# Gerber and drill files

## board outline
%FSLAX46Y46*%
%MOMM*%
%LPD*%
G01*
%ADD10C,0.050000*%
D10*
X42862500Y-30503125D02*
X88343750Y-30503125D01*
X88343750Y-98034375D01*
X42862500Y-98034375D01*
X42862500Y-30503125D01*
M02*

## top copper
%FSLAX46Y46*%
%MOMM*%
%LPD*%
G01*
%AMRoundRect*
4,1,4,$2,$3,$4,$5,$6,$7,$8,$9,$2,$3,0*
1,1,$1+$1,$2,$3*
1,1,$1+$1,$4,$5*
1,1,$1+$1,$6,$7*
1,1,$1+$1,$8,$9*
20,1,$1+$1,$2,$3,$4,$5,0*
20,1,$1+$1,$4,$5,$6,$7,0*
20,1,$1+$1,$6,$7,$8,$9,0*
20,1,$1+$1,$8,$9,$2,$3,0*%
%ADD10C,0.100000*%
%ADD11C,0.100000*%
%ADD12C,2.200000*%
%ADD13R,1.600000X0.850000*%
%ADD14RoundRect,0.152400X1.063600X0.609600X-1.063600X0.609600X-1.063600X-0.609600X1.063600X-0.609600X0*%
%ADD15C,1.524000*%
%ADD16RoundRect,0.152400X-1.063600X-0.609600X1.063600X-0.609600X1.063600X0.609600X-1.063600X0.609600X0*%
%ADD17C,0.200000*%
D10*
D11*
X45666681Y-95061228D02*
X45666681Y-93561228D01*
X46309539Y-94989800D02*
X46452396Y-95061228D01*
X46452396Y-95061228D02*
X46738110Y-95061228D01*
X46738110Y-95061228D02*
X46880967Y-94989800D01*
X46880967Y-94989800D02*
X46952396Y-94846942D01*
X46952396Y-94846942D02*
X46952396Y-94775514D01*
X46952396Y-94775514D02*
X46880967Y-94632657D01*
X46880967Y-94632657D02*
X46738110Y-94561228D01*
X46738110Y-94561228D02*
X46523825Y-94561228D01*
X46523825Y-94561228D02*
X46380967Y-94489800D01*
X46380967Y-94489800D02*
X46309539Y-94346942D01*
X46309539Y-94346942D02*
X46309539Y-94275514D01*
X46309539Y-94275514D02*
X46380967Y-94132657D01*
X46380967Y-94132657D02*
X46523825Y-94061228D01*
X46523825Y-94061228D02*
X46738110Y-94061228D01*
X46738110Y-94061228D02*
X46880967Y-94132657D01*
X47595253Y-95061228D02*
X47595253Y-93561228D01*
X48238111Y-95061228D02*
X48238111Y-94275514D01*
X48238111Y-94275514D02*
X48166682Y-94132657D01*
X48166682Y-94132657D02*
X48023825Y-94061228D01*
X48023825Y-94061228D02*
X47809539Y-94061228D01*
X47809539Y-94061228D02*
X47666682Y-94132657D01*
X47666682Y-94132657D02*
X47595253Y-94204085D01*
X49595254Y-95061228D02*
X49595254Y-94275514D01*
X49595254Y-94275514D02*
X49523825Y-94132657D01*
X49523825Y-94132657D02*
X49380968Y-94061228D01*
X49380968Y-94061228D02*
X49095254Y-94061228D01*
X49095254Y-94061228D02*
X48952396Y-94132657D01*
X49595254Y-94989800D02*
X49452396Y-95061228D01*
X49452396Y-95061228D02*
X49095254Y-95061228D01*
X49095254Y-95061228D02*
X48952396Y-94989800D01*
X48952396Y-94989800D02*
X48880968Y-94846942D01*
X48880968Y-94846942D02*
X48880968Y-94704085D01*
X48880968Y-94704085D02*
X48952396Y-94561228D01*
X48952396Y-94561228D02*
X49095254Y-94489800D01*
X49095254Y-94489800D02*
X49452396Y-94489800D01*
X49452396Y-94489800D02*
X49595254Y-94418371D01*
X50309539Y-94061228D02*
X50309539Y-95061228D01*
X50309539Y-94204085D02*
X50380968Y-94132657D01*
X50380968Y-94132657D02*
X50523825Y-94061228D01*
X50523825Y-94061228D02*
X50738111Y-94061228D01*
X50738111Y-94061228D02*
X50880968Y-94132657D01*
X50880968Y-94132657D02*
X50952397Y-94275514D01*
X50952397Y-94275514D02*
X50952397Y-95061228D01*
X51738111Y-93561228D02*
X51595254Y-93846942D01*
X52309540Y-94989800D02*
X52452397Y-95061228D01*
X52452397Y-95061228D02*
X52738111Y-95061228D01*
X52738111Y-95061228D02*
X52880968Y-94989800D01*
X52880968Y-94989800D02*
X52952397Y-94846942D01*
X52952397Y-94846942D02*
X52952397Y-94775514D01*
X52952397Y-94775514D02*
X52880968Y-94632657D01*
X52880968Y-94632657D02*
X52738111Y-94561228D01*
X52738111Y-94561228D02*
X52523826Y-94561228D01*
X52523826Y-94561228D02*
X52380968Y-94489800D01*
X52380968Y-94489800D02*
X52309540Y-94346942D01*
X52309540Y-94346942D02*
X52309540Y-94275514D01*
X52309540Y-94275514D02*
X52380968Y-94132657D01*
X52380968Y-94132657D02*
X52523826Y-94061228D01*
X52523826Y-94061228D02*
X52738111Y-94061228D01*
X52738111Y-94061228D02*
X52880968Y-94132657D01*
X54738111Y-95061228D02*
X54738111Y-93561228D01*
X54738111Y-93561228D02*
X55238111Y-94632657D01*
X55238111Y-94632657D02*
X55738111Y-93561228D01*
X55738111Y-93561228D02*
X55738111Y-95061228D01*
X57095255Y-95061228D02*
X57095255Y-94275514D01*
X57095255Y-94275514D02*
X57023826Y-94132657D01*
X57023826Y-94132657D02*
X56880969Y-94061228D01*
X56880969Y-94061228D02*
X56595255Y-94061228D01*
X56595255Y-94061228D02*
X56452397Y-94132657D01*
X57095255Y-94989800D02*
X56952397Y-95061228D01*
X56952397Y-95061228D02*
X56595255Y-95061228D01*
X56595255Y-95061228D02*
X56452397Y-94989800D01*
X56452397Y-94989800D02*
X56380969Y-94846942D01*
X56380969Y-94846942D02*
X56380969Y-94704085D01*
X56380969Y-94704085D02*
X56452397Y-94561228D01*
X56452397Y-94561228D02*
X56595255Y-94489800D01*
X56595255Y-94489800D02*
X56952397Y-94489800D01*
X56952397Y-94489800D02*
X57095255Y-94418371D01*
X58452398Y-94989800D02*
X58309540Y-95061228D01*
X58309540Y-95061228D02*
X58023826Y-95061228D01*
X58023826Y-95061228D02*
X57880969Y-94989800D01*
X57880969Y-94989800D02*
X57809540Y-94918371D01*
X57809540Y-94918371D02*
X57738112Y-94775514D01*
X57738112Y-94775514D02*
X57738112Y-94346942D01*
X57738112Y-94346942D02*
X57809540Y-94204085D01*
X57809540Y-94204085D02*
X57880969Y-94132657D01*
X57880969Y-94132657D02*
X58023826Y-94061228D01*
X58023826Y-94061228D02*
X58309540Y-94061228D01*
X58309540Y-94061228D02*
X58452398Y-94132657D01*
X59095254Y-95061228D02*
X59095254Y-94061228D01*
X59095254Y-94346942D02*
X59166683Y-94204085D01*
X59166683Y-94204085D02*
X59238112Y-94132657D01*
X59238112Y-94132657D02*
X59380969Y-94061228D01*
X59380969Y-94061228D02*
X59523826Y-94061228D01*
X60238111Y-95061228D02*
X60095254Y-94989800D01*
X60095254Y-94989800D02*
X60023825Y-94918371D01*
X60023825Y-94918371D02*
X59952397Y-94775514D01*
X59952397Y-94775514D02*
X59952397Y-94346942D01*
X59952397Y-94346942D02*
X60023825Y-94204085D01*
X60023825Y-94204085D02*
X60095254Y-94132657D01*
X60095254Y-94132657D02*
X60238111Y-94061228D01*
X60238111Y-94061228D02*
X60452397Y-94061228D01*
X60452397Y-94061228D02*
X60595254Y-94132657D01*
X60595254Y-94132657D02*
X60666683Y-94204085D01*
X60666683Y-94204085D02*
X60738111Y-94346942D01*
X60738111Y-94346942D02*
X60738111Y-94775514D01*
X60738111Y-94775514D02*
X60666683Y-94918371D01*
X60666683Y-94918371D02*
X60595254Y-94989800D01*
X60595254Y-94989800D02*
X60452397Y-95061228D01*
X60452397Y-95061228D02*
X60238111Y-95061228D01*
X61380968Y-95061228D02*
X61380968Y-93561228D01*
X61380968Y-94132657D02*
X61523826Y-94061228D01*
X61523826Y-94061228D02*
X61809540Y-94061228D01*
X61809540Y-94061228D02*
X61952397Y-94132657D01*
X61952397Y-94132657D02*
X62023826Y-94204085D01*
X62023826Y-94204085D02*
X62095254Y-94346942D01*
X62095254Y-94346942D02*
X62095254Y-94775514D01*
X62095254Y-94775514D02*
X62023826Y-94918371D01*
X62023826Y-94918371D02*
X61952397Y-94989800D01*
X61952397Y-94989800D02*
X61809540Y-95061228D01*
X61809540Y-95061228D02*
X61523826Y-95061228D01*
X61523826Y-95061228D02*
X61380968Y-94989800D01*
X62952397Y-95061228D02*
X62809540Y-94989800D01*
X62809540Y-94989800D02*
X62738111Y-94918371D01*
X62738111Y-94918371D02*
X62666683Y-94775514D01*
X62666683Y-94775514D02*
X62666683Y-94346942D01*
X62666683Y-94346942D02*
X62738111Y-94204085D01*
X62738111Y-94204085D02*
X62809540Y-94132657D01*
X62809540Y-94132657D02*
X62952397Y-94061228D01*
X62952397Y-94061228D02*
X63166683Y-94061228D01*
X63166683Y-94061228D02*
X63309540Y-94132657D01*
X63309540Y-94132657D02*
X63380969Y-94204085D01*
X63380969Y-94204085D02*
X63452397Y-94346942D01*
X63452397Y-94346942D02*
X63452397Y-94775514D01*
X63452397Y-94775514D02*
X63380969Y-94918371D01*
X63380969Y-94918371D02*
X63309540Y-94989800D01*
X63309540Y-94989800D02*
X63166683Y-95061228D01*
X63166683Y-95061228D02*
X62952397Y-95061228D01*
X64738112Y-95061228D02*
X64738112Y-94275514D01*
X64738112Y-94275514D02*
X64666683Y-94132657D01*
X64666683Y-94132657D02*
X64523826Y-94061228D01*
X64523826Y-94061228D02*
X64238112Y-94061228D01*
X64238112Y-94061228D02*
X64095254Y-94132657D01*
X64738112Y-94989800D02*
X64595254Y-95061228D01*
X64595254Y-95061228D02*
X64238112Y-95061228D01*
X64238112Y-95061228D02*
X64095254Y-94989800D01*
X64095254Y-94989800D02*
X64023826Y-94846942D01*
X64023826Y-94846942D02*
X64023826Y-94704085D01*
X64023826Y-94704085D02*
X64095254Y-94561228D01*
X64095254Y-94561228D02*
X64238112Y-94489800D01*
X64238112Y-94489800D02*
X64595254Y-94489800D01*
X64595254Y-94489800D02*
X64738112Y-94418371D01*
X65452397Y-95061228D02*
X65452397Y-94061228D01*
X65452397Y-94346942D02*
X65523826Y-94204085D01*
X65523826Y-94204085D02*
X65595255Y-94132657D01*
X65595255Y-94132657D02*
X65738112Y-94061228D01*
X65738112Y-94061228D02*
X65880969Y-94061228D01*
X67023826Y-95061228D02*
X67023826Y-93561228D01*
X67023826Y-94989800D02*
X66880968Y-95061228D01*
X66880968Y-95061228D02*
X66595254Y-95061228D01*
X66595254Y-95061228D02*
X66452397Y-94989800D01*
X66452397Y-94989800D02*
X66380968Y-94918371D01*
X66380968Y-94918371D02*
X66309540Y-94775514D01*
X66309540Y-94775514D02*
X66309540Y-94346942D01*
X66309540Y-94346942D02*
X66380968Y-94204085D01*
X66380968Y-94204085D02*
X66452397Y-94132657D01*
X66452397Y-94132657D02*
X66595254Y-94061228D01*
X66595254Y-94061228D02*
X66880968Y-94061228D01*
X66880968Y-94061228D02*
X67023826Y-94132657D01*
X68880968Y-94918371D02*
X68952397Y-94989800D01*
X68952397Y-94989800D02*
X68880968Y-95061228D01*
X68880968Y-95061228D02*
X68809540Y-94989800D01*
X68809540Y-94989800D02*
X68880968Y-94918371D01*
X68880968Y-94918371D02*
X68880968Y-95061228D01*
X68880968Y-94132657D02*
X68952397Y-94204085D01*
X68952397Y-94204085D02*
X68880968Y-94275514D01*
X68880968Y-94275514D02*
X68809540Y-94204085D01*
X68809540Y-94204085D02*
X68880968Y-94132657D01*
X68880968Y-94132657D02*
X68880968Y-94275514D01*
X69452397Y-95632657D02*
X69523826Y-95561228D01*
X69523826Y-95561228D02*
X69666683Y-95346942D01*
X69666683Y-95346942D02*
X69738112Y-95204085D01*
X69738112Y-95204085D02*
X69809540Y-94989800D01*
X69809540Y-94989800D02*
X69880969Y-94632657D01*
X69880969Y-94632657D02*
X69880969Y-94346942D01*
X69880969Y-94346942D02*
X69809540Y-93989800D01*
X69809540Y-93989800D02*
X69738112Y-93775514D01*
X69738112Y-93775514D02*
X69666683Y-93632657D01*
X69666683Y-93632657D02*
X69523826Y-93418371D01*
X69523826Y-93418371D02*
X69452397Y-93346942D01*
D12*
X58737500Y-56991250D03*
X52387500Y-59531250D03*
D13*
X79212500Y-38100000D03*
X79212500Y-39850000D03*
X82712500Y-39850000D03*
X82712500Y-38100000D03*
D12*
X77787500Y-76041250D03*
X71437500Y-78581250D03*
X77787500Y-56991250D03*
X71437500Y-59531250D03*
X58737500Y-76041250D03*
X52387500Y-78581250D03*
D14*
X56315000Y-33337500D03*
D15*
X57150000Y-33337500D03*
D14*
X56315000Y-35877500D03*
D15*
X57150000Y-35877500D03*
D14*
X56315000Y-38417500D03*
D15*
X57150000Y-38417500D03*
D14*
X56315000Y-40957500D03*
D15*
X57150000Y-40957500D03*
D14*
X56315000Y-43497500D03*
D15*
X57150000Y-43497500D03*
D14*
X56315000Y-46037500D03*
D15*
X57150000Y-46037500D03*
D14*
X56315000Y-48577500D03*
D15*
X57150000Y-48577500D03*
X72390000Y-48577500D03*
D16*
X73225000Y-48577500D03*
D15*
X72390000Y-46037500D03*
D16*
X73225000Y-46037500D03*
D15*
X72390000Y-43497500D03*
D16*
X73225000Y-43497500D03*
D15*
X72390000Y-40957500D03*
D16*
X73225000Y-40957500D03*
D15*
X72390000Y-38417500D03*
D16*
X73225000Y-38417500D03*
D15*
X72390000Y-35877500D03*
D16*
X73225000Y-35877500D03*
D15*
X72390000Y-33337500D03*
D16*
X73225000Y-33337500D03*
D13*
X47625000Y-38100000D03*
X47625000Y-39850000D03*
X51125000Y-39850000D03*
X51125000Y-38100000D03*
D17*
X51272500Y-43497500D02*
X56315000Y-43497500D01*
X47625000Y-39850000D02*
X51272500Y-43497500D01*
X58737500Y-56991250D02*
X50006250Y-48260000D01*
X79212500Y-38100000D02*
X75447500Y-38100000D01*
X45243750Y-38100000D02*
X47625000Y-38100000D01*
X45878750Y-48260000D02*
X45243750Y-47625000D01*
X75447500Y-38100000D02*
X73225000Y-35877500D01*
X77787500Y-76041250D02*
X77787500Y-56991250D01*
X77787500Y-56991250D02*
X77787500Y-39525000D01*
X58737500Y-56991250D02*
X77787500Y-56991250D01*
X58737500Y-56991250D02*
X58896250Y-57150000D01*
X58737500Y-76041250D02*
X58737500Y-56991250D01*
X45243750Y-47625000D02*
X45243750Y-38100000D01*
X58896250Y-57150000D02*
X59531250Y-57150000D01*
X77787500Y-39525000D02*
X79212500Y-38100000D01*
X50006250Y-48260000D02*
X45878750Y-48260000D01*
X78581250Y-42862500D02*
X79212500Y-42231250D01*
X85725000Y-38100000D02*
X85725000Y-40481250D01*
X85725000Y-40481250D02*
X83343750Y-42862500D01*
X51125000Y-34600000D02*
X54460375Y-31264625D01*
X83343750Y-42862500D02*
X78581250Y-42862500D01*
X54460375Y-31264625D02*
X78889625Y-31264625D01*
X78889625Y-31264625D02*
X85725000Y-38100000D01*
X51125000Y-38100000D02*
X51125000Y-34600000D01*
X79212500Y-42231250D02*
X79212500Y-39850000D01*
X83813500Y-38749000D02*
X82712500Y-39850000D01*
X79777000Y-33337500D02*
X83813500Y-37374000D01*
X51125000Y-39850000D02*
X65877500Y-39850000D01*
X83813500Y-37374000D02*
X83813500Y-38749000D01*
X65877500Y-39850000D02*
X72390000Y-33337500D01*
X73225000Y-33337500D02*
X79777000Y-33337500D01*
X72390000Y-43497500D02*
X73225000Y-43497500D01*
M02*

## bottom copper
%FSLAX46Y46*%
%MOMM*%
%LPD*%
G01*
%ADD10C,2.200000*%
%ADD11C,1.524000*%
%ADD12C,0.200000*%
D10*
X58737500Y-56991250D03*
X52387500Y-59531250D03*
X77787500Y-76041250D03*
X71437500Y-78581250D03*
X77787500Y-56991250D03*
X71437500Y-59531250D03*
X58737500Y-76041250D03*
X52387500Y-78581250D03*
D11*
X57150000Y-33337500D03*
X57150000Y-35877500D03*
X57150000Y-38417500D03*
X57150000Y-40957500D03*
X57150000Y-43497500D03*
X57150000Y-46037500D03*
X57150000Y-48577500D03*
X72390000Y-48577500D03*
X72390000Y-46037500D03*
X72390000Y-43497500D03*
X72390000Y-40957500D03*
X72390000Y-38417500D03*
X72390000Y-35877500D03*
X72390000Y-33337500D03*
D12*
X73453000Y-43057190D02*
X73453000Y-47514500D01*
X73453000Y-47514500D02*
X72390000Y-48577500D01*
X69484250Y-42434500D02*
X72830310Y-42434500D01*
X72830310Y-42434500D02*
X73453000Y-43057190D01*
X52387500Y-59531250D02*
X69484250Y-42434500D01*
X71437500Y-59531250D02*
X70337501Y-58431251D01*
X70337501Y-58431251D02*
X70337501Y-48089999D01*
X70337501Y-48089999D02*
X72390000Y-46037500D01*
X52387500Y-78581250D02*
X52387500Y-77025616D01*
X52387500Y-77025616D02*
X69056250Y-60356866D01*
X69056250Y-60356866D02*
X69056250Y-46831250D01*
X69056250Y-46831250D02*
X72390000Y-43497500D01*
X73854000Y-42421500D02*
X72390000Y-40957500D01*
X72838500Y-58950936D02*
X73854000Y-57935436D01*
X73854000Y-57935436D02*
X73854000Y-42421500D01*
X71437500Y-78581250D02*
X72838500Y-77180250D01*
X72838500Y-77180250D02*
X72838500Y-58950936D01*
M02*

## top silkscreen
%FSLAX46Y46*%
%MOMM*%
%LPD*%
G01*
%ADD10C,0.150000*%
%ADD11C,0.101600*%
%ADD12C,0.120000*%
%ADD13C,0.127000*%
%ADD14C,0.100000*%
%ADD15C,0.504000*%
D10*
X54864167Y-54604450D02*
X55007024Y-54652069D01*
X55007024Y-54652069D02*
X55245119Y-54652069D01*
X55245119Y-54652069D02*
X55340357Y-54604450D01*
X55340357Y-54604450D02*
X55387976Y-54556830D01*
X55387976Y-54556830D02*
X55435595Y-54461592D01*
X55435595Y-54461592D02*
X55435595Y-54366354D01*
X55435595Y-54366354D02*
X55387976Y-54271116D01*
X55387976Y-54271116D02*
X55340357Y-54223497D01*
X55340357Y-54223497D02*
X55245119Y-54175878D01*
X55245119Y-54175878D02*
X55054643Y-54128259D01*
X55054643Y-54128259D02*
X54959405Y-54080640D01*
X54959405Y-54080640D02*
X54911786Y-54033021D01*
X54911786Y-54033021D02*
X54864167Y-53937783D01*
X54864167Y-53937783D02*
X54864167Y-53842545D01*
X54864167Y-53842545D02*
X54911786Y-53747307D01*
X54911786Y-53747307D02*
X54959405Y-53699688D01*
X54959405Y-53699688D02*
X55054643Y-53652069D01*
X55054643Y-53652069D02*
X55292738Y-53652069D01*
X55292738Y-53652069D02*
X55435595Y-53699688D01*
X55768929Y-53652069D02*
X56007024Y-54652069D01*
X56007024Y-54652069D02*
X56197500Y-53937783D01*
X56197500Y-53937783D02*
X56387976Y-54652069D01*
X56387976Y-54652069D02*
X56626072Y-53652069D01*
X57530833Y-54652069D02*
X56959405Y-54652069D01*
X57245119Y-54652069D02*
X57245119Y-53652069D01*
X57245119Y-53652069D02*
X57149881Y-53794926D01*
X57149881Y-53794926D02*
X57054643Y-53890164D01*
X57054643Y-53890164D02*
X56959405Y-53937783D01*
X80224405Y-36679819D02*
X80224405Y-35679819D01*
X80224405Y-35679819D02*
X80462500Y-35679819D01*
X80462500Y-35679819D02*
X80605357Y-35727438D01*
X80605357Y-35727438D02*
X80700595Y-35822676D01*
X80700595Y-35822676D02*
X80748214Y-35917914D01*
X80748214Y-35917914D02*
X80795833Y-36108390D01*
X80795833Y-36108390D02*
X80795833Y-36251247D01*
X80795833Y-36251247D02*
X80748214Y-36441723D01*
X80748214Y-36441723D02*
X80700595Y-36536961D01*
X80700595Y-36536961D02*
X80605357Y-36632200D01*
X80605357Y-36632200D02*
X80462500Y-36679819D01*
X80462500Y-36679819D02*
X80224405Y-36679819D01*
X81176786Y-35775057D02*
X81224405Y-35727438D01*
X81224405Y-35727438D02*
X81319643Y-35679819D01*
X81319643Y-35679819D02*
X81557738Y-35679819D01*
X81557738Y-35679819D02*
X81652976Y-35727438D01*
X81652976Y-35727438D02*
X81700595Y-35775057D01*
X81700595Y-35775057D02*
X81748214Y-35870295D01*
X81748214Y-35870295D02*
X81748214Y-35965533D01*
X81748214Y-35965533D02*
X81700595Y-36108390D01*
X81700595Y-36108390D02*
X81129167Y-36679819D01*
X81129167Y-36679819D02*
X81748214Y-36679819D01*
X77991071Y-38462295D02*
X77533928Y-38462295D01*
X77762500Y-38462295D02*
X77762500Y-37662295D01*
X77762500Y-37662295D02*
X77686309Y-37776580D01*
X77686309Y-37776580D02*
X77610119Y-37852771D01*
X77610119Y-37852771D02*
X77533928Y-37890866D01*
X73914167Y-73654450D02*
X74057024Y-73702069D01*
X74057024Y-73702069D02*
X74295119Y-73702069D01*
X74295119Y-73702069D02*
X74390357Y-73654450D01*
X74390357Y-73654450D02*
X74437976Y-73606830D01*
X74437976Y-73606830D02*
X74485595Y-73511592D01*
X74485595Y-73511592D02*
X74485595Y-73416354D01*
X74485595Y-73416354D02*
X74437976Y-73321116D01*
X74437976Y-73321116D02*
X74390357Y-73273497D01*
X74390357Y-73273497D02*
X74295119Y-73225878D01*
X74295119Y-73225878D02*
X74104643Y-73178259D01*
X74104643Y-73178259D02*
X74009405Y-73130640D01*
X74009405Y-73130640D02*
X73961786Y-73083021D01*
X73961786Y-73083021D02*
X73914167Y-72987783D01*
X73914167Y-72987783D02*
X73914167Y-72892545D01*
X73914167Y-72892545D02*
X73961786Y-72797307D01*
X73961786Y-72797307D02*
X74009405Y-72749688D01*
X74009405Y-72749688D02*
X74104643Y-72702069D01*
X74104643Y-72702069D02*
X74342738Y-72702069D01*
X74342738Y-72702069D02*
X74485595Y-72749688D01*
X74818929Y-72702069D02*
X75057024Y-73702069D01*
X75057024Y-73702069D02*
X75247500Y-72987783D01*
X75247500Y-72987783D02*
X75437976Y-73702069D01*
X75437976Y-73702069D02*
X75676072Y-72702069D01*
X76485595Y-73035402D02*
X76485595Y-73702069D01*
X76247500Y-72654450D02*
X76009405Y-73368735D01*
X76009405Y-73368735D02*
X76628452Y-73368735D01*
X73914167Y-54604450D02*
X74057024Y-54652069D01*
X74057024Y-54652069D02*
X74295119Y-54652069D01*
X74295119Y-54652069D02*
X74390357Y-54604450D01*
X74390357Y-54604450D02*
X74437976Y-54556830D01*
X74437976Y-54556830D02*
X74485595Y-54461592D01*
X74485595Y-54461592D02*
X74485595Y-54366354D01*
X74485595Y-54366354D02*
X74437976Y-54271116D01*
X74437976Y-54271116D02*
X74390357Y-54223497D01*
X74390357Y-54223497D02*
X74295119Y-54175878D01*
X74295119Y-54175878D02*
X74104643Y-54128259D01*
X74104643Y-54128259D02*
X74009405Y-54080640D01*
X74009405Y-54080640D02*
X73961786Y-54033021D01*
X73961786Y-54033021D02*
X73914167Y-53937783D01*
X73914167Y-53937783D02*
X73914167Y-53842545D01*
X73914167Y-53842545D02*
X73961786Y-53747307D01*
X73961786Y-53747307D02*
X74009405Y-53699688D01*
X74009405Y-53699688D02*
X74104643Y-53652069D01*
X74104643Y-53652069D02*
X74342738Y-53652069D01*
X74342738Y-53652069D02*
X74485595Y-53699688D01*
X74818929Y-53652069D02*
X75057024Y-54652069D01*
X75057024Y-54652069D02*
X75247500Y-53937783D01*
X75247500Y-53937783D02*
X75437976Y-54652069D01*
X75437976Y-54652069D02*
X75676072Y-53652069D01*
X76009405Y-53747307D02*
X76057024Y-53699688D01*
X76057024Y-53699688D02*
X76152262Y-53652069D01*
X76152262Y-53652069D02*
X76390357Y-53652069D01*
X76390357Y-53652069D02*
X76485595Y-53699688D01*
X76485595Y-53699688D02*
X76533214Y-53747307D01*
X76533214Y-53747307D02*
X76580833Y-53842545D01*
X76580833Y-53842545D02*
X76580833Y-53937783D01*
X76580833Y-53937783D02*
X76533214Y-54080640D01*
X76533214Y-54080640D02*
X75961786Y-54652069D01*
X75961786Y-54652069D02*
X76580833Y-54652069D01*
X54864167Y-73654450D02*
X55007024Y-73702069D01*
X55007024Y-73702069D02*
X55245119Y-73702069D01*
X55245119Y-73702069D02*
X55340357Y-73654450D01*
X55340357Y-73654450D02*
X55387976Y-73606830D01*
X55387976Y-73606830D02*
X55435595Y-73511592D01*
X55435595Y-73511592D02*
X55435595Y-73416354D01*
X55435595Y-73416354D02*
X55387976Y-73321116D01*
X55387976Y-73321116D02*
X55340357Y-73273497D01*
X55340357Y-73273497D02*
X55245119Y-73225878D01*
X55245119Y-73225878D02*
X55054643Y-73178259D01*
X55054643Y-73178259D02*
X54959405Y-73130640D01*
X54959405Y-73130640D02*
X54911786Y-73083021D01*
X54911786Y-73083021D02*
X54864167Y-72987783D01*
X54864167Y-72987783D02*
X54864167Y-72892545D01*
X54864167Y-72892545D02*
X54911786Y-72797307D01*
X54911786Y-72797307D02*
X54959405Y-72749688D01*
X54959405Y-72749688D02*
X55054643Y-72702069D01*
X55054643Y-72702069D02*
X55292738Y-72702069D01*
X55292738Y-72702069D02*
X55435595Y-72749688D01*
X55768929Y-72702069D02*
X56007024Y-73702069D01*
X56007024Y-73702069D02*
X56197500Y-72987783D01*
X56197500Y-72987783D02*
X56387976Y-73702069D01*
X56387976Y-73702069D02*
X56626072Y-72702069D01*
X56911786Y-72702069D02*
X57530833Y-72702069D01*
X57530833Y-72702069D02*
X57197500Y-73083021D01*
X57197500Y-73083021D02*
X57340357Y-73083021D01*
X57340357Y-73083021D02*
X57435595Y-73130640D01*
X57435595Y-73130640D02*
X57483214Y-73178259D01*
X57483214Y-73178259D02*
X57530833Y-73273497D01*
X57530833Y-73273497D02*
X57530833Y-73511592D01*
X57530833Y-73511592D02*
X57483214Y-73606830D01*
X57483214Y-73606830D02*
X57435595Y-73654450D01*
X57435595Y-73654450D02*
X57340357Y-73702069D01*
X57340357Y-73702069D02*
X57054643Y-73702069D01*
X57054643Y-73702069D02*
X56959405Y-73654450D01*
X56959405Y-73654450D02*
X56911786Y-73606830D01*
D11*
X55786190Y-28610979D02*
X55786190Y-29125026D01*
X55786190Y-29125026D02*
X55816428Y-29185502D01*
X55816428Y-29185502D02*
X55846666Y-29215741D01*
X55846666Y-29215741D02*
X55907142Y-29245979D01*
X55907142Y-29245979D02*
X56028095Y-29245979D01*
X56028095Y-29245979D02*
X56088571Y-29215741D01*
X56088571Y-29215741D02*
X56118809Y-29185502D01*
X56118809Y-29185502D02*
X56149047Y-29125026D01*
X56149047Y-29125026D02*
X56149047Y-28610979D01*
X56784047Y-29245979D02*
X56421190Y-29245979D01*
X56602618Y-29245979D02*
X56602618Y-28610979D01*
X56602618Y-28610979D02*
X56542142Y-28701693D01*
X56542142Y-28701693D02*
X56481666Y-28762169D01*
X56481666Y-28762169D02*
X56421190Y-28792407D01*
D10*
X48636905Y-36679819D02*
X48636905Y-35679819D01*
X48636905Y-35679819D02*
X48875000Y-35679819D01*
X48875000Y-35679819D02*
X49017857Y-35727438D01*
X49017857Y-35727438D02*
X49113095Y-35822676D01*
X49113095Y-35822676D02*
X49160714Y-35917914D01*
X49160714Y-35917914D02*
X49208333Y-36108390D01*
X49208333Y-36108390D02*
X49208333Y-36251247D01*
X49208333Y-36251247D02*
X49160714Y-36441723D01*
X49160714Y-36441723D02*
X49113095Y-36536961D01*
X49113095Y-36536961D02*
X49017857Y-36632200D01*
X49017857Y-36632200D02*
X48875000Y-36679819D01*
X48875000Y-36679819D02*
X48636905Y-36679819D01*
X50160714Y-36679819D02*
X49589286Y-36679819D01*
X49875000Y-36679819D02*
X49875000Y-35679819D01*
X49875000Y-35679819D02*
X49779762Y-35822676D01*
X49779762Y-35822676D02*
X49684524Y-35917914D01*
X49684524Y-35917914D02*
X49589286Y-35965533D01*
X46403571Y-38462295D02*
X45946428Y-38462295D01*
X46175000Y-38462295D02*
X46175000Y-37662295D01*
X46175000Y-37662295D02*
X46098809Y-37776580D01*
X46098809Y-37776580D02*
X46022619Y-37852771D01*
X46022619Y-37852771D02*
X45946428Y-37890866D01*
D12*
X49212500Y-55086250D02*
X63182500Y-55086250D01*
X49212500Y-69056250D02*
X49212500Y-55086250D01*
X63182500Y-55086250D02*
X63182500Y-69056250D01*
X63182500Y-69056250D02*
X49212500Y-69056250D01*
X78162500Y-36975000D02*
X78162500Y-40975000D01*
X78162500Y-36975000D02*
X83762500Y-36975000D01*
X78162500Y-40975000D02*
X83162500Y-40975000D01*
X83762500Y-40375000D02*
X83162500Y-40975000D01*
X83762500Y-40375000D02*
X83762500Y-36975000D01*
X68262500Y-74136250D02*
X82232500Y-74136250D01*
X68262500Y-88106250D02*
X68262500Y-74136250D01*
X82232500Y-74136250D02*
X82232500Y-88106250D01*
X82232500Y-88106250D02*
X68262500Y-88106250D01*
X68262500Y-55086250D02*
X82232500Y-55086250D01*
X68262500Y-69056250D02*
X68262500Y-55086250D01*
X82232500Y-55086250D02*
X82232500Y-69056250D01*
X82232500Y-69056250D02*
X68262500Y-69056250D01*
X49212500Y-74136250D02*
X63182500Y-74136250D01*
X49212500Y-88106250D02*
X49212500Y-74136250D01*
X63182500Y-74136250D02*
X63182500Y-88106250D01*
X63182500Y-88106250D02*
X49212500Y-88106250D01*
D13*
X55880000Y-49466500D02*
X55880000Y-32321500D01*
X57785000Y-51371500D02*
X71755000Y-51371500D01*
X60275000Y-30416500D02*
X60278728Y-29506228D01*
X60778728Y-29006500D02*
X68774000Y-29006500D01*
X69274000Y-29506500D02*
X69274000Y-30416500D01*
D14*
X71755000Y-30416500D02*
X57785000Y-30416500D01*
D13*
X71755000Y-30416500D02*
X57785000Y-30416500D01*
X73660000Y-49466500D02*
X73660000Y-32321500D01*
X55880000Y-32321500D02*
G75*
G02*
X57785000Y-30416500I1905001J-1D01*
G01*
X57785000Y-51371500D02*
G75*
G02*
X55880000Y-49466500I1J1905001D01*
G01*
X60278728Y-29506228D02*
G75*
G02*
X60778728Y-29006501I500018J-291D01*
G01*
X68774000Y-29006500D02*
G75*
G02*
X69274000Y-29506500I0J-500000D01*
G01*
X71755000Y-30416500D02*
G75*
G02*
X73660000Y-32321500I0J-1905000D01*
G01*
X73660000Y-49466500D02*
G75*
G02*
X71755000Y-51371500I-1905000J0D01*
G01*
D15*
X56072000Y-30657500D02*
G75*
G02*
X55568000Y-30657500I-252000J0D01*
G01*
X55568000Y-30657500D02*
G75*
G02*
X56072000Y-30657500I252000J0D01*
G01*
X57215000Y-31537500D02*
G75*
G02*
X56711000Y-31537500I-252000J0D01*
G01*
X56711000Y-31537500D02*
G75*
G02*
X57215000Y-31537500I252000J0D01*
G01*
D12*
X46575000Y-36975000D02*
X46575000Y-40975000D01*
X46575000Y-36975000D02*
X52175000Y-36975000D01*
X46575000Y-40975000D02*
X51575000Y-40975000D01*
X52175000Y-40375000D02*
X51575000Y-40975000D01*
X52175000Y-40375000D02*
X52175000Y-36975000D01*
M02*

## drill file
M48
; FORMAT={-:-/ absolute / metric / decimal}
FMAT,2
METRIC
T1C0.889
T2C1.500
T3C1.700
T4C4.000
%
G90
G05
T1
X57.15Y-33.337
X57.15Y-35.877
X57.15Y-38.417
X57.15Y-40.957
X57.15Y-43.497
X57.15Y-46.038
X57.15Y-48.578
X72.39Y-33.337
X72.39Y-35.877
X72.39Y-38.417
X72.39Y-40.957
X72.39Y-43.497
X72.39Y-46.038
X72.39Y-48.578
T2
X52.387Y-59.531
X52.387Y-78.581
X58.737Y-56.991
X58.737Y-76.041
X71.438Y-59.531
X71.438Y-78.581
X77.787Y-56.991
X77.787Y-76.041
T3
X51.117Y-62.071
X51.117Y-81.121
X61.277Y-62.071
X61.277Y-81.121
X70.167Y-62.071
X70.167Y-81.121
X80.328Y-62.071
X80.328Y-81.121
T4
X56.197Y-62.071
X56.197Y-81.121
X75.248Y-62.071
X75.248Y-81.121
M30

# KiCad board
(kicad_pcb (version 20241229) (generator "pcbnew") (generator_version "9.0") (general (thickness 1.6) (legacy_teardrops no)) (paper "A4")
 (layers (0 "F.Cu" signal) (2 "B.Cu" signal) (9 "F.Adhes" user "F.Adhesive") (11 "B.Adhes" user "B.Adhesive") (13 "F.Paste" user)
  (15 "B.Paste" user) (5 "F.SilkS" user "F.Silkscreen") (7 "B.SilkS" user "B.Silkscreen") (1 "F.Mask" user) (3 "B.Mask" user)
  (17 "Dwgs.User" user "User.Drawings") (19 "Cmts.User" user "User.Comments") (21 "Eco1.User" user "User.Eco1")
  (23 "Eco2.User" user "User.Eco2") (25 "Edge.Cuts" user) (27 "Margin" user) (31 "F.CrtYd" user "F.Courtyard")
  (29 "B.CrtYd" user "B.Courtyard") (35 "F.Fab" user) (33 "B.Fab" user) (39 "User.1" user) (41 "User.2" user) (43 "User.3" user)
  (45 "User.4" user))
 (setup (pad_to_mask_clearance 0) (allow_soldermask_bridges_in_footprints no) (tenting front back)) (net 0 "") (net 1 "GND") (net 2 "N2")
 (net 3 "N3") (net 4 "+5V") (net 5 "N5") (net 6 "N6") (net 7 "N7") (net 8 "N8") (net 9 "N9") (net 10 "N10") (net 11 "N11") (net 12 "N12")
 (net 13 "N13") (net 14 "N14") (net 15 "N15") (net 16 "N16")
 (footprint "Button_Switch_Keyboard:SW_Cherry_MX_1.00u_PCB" (layer "F.Cu") (at 58.7375 56.99125)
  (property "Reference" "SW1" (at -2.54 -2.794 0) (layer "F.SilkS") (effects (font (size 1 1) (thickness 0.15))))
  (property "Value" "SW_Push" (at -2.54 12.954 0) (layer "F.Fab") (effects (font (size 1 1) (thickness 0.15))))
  (fp_line (start -9.525 -1.905) (end 4.445 -1.905) (stroke (width 0.12) (type solid)) (layer "F.SilkS"))
  (fp_line (start -9.525 12.065) (end -9.525 -1.905) (stroke (width 0.12) (type solid)) (layer "F.SilkS"))
  (fp_line (start 4.445 -1.905) (end 4.445 12.065) (stroke (width 0.12) (type solid)) (layer "F.SilkS"))
  (fp_line (start 4.445 12.065) (end -9.525 12.065) (stroke (width 0.12) (type solid)) (layer "F.SilkS"))
  (pad "" np_thru_hole circle (at -7.62 5.08) (size 1.7 1.7) (drill 1.7) (layers "*.Cu" "*.Mask"))
  (pad "" np_thru_hole circle (at -2.54 5.08) (size 4 4) (drill 4) (layers "*.Cu" "*.Mask"))
  (pad "" np_thru_hole circle (at 2.54 5.08) (size 1.7 1.7) (drill 1.7) (layers "*.Cu" "*.Mask"))
  (pad "1" thru_hole circle (at 0 0) (size 2.2 2.2) (drill 1.5) (layers "*.Cu" "*.Mask") (remove_unused_layers no) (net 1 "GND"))
  (pad "2" thru_hole circle (at -6.35 2.54) (size 2.2 2.2) (drill 1.5) (layers "*.Cu" "*.Mask") (remove_unused_layers no) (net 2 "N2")))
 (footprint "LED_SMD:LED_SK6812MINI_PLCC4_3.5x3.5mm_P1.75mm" (layer "F.Cu") (at 80.9625 38.975)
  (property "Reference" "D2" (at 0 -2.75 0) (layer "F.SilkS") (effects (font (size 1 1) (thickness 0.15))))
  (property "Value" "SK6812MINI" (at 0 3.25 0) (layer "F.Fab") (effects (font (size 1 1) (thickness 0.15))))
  (fp_line (start -2.8 -2) (end -2.8 2) (stroke (width 0.12) (type default)) (layer "F.SilkS"))
  (fp_line (start -2.8 -2) (end 2.8 -2) (stroke (width 0.12) (type solid)) (layer "F.SilkS"))
  (fp_line (start -2.8 2) (end 2.2 2) (stroke (width 0.12) (type solid)) (layer "F.SilkS"))
  (fp_line (start 2.8 1.4) (end 2.2 2) (stroke (width 0.12) (type default)) (layer "F.SilkS"))
  (fp_line (start 2.8 1.4) (end 2.8 -2) (stroke (width 0.12) (type solid)) (layer "F.SilkS"))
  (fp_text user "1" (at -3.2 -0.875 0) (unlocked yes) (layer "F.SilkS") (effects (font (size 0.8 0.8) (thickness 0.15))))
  (pad "1" smd rect (at -1.75 -0.875) (size 1.6 0.85) (layers "F.Cu" "F.Mask" "F.Paste") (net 1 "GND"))
  (pad "2" smd rect (at -1.75 0.875) (size 1.6 0.85) (layers "F.Cu" "F.Mask" "F.Paste") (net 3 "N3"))
  (pad "3" smd rect (at 1.75 0.875) (size 1.6 0.85) (layers "F.Cu" "F.Mask" "F.Paste") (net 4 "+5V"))
  (pad "4" smd rect (at 1.75 -0.875) (size 1.6 0.85) (layers "F.Cu" "F.Mask" "F.Paste") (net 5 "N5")))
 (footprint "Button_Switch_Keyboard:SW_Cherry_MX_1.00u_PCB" (layer "F.Cu") (at 77.7875 76.04125)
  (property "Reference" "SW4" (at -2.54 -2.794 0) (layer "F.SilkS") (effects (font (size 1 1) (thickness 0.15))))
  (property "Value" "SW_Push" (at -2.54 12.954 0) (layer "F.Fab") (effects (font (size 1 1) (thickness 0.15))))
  (fp_line (start -9.525 -1.905) (end 4.445 -1.905) (stroke (width 0.12) (type solid)) (layer "F.SilkS"))
  (fp_line (start -9.525 12.065) (end -9.525 -1.905) (stroke (width 0.12) (type solid)) (layer "F.SilkS"))
  (fp_line (start 4.445 -1.905) (end 4.445 12.065) (stroke (width 0.12) (type solid)) (layer "F.SilkS"))
  (fp_line (start 4.445 12.065) (end -9.525 12.065) (stroke (width 0.12) (type solid)) (layer "F.SilkS"))
  (pad "" np_thru_hole circle (at -7.62 5.08) (size 1.7 1.7) (drill 1.7) (layers "*.Cu" "*.Mask"))
  (pad "" np_thru_hole circle (at -2.54 5.08) (size 4 4) (drill 4) (layers "*.Cu" "*.Mask"))
  (pad "" np_thru_hole circle (at 2.54 5.08) (size 1.7 1.7) (drill 1.7) (layers "*.Cu" "*.Mask"))
  (pad "1" thru_hole circle (at 0 0) (size 2.2 2.2) (drill 1.5) (layers "*.Cu" "*.Mask") (remove_unused_layers no) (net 1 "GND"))
  (pad "2" thru_hole circle (at -6.35 2.54) (size 2.2 2.2) (drill 1.5) (layers "*.Cu" "*.Mask") (remove_unused_layers no) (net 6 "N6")))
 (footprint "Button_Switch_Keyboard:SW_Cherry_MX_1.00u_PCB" (layer "F.Cu") (at 77.7875 56.99125)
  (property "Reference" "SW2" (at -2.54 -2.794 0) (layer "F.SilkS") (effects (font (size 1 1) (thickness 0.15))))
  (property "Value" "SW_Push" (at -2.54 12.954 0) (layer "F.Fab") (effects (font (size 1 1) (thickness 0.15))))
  (fp_line (start -9.525 -1.905) (end 4.445 -1.905) (stroke (width 0.12) (type solid)) (layer "F.SilkS"))
  (fp_line (start -9.525 12.065) (end -9.525 -1.905) (stroke (width 0.12) (type solid)) (layer "F.SilkS"))
  (fp_line (start 4.445 -1.905) (end 4.445 12.065) (stroke (width 0.12) (type solid)) (layer "F.SilkS"))
  (fp_line (start 4.445 12.065) (end -9.525 12.065) (stroke (width 0.12) (type solid)) (layer "F.SilkS"))
  (pad "" np_thru_hole circle (at -7.62 5.08) (size 1.7 1.7) (drill 1.7) (layers "*.Cu" "*.Mask"))
  (pad "" np_thru_hole circle (at -2.54 5.08) (size 4 4) (drill 4) (layers "*.Cu" "*.Mask"))
  (pad "" np_thru_hole circle (at 2.54 5.08) (size 1.7 1.7) (drill 1.7) (layers "*.Cu" "*.Mask"))
  (pad "1" thru_hole circle (at 0 0) (size 2.2 2.2) (drill 1.5) (layers "*.Cu" "*.Mask") (remove_unused_layers no) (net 1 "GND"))
  (pad "2" thru_hole circle (at -6.35 2.54) (size 2.2 2.2) (drill 1.5) (layers "*.Cu" "*.Mask") (remove_unused_layers no) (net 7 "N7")))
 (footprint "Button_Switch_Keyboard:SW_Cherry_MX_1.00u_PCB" (layer "F.Cu") (at 58.7375 76.04125)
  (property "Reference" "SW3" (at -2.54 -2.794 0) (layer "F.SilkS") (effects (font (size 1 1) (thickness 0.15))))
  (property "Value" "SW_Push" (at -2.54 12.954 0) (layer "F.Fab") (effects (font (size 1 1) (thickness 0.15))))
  (fp_line (start -9.525 -1.905) (end 4.445 -1.905) (stroke (width 0.12) (type solid)) (layer "F.SilkS"))
  (fp_line (start -9.525 12.065) (end -9.525 -1.905) (stroke (width 0.12) (type solid)) (layer "F.SilkS"))
  (fp_line (start 4.445 -1.905) (end 4.445 12.065) (stroke (width 0.12) (type solid)) (layer "F.SilkS"))
  (fp_line (start 4.445 12.065) (end -9.525 12.065) (stroke (width 0.12) (type solid)) (layer "F.SilkS"))
  (pad "" np_thru_hole circle (at -7.62 5.08) (size 1.7 1.7) (drill 1.7) (layers "*.Cu" "*.Mask"))
  (pad "" np_thru_hole circle (at -2.54 5.08) (size 4 4) (drill 4) (layers "*.Cu" "*.Mask"))
  (pad "" np_thru_hole circle (at 2.54 5.08) (size 1.7 1.7) (drill 1.7) (layers "*.Cu" "*.Mask"))
  (pad "1" thru_hole circle (at 0 0) (size 2.2 2.2) (drill 1.5) (layers "*.Cu" "*.Mask") (remove_unused_layers no) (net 1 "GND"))
  (pad "2" thru_hole circle (at -6.35 2.54) (size 2.2 2.2) (drill 1.5) (layers "*.Cu" "*.Mask") (remove_unused_layers no) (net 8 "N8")))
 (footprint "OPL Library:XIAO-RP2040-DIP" (layer "F.Cu") (at 64.77 40.9575)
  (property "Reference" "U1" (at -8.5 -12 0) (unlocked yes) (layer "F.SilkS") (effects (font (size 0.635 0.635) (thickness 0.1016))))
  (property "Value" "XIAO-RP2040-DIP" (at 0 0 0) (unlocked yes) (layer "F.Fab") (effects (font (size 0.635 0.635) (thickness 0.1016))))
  (fp_line (start -8.89 8.509) (end -8.89 -8.636) (stroke (width 0.127) (type solid)) (layer "F.SilkS"))
  (fp_line (start -6.985 10.414) (end 6.985 10.414) (stroke (width 0.127) (type solid)) (layer "F.SilkS"))
  (fp_line (start -4.495 -10.541) (end -4.491272 -11.451272) (stroke (width 0.127) (type solid)) (layer "F.SilkS"))
  (fp_line (start -3.991272 -11.951) (end 4.004 -11.951) (stroke (width 0.127) (type solid)) (layer "F.SilkS"))
  (fp_line (start 4.504 -11.451) (end 4.504 -10.541) (stroke (width 0.127) (type solid)) (layer "F.SilkS"))
  (fp_line (start 6.985 -10.541) (end -6.985 -10.541) (stroke (width 0.1) (type solid)) (layer "F.SilkS"))
  (fp_line (start 6.985 -10.541) (end -6.985 -10.541) (stroke (width 0.127) (type solid)) (layer "F.SilkS"))
  (fp_line (start 8.89 8.509) (end 8.89 -8.636) (stroke (width 0.127) (type solid)) (layer "F.SilkS"))
  (fp_arc (start -8.89 -8.636) (mid -8.332038 -9.983038) (end -6.985 -10.541) (stroke (width 0.127) (type solid)) (layer "F.SilkS"))
  (fp_arc (start -6.985 10.414) (mid -8.332038 9.856038) (end -8.89 8.509) (stroke (width 0.127) (type solid)) (layer "F.SilkS"))
  (fp_arc (start -4.491272 -11.451272) (mid -4.344728 -11.80464) (end -3.991272 -11.951) (stroke (width 0.127) (type default))
   (layer "F.SilkS"))
  (fp_arc (start 4.004 -11.951) (mid 4.357553 -11.804553) (end 4.504 -11.451) (stroke (width 0.127) (type default)) (layer "F.SilkS"))
  (fp_arc (start 6.985 -10.541) (mid 8.332038 -9.983038) (end 8.89 -8.636) (stroke (width 0.127) (type solid)) (layer "F.SilkS"))
  (fp_arc (start 8.89 8.509) (mid 8.332038 9.856038) (end 6.985 10.414) (stroke (width 0.127) (type solid)) (layer "F.SilkS"))
  (fp_circle (center -8.95 -10.3) (end -8.95 -10.554) (stroke (width 0.5) (type solid)) (fill yes) (layer "F.SilkS"))
  (fp_circle (center -7.807 -9.42) (end -7.807 -9.674) (stroke (width 0.5) (type solid)) (fill yes) (layer "F.SilkS"))
  (pad "1" smd roundrect (at -8.455 -7.62 180) (size 2.432 1.524) (layers "F.Cu" "F.Mask") (roundrect_rratio 0.1) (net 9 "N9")
   (thermal_bridge_angle 45))
  (pad "1" thru_hole circle (at -7.62 -7.62 180) (size 1.524 1.524) (drill 0.889) (layers "*.Cu" "*.Mask") (remove_unused_layers no)
   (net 9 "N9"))
  (pad "2" smd roundrect (at -8.455 -5.08 180) (size 2.432 1.524) (layers "F.Cu" "F.Mask") (roundrect_rratio 0.1) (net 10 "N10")
   (thermal_bridge_angle 45))
  (pad "2" thru_hole circle (at -7.62 -5.08 180) (size 1.524 1.524) (drill 0.889) (layers "*.Cu" "*.Mask") (remove_unused_layers no)
   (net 10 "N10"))
  (pad "3" smd roundrect (at -8.455 -2.54 180) (size 2.432 1.524) (layers "F.Cu" "F.Mask") (roundrect_rratio 0.1) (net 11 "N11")
   (thermal_bridge_angle 45))
  (pad "3" thru_hole circle (at -7.62 -2.54 180) (size 1.524 1.524) (drill 0.889) (layers "*.Cu" "*.Mask") (remove_unused_layers no)
   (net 11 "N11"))
  (pad "4" smd roundrect (at -8.455 0 180) (size 2.432 1.524) (layers "F.Cu" "F.Mask") (roundrect_rratio 0.1) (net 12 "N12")
   (thermal_bridge_angle 45))
  (pad "4" thru_hole circle (at -7.62 0 180) (size 1.524 1.524) (drill 0.889) (layers "*.Cu" "*.Mask") (remove_unused_layers no)
   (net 12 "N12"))
  (pad "5" smd roundrect (at -8.455 2.54 180) (size 2.432 1.524) (layers "F.Cu" "F.Mask") (roundrect_rratio 0.1) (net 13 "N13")
   (thermal_bridge_angle 45))
  (pad "5" thru_hole circle (at -7.62 2.54 180) (size 1.524 1.524) (drill 0.889) (layers "*.Cu" "*.Mask") (remove_unused_layers no)
   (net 13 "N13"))
  (pad "6" smd roundrect (at -8.455 5.08 180) (size 2.432 1.524) (layers "F.Cu" "F.Mask") (roundrect_rratio 0.1) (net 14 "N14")
   (thermal_bridge_angle 45))
  (pad "6" thru_hole circle (at -7.62 5.08 180) (size 1.524 1.524) (drill 0.889) (layers "*.Cu" "*.Mask") (remove_unused_layers no)
   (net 14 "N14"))
  (pad "7" smd roundrect (at -8.455 7.62 180) (size 2.432 1.524) (layers "F.Cu" "F.Mask") (roundrect_rratio 0.1) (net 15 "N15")
   (thermal_bridge_angle 45))
  (pad "7" thru_hole circle (at -7.62 7.62 180) (size 1.524 1.524) (drill 0.889) (layers "*.Cu" "*.Mask") (remove_unused_layers no)
   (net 15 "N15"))
  (pad "8" thru_hole circle (at 7.62 7.62) (size 1.524 1.524) (drill 0.889) (layers "*.Cu" "*.Mask") (remove_unused_layers no) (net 2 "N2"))
  (pad "8" smd roundrect (at 8.455 7.62) (size 2.432 1.524) (layers "F.Cu" "F.Mask") (roundrect_rratio 0.1) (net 2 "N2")
   (thermal_bridge_angle 45))
  (pad "9" thru_hole circle (at 7.62 5.08) (size 1.524 1.524) (drill 0.889) (layers "*.Cu" "*.Mask") (remove_unused_layers no) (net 7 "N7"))
  (pad "9" smd roundrect (at 8.455 5.08) (size 2.432 1.524) (layers "F.Cu" "F.Mask") (roundrect_rratio 0.1) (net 7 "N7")
   (thermal_bridge_angle 45))
  (pad "10" thru_hole circle (at 7.62 2.54) (size 1.524 1.524) (drill 0.889) (layers "*.Cu" "*.Mask") (remove_unused_layers no) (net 8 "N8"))
  (pad "10" smd roundrect (at 8.455 2.54) (size 2.432 1.524) (layers "F.Cu" "F.Mask") (roundrect_rratio 0.1) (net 8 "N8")
   (thermal_bridge_angle 45))
  (pad "11" thru_hole circle (at 7.62 0) (size 1.524 1.524) (drill 0.889) (layers "*.Cu" "*.Mask") (remove_unused_layers no) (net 6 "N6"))
  (pad "11" smd roundrect (at 8.455 0) (size 2.432 1.524) (layers "F.Cu" "F.Mask") (roundrect_rratio 0.1) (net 6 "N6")
   (thermal_bridge_angle 45))
  (pad "12" thru_hole circle (at 7.62 -2.54) (size 1.524 1.524) (drill 0.889) (layers "*.Cu" "*.Mask") (remove_unused_layers no)
   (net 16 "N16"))
  (pad "12" smd roundrect (at 8.455 -2.54) (size 2.432 1.524) (layers "F.Cu" "F.Mask") (roundrect_rratio 0.1) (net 16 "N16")
   (thermal_bridge_angle 45))
  (pad "13" thru_hole circle (at 7.62 -5.08) (size 1.524 1.524) (drill 0.889) (layers "*.Cu" "*.Mask") (remove_unused_layers no)
   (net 1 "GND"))
  (pad "13" smd roundrect (at 8.455 -5.08) (size 2.432 1.524) (layers "F.Cu" "F.Mask") (roundrect_rratio 0.1) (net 1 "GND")
   (thermal_bridge_angle 45))
  (pad "14" thru_hole circle (at 7.62 -7.62) (size 1.524 1.524) (drill 0.889) (layers "*.Cu" "*.Mask") (remove_unused_layers no)
   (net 4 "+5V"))
  (pad "14" smd roundrect (at 8.455 -7.62) (size 2.432 1.524) (layers "F.Cu" "F.Mask") (roundrect_rratio 0.1) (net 4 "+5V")
   (thermal_bridge_angle 45)))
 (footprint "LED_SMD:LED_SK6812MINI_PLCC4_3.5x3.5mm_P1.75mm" (layer "F.Cu") (at 49.375 38.975)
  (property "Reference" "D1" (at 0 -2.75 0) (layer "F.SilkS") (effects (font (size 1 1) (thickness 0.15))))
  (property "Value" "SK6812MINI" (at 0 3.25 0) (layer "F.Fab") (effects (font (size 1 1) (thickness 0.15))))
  (fp_line (start -2.8 -2) (end -2.8 2) (stroke (width 0.12) (type default)) (layer "F.SilkS"))
  (fp_line (start -2.8 -2) (end 2.8 -2) (stroke (width 0.12) (type solid)) (layer "F.SilkS"))
  (fp_line (start -2.8 2) (end 2.2 2) (stroke (width 0.12) (type solid)) (layer "F.SilkS"))
  (fp_line (start 2.8 1.4) (end 2.2 2) (stroke (width 0.12) (type default)) (layer "F.SilkS"))
  (fp_line (start 2.8 1.4) (end 2.8 -2) (stroke (width 0.12) (type solid)) (layer "F.SilkS"))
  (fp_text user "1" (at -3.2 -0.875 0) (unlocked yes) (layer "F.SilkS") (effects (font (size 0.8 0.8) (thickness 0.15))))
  (pad "1" smd rect (at -1.75 -0.875) (size 1.6 0.85) (layers "F.Cu" "F.Mask" "F.Paste") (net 1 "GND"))
  (pad "2" smd rect (at -1.75 0.875) (size 1.6 0.85) (layers "F.Cu" "F.Mask" "F.Paste") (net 13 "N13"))
  (pad "3" smd rect (at 1.75 0.875) (size 1.6 0.85) (layers "F.Cu" "F.Mask" "F.Paste") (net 4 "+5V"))
  (pad "4" smd rect (at 1.75 -0.875) (size 1.6 0.85) (layers "F.Cu" "F.Mask" "F.Paste") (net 3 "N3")))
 (gr_rect (start 42.8625 30.503125) (end 88.34375 98.034375) (stroke (width 0.05) (type solid)) (fill no) (layer "Edge.Cuts"))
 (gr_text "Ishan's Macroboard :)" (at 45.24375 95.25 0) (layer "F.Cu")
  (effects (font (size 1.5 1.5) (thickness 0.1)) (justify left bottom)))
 (segment (start 51.2725 43.4975) (end 56.315 43.4975) (width 0.2) (layer "F.Cu") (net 13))
 (segment (start 47.625 39.85) (end 51.2725 43.4975) (width 0.2) (layer "F.Cu") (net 13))
 (segment (start 58.7375 56.99125) (end 50.00625 48.26) (width 0.2) (layer "F.Cu") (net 1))
 (segment (start 79.2125 38.1) (end 75.4475 38.1) (width 0.2) (layer "F.Cu") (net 1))
 (segment (start 45.24375 38.1) (end 47.625 38.1) (width 0.2) (layer "F.Cu") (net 1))
 (segment (start 45.87875 48.26) (end 45.24375 47.625) (width 0.2) (layer "F.Cu") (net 1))
 (segment (start 75.4475 38.1) (end 73.225 35.8775) (width 0.2) (layer "F.Cu") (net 1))
 (segment (start 77.7875 76.04125) (end 77.7875 56.99125) (width 0.2) (layer "F.Cu") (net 1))
 (segment (start 77.7875 56.99125) (end 77.7875 39.525) (width 0.2) (layer "F.Cu") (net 1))
 (segment (start 58.7375 56.99125) (end 77.7875 56.99125) (width 0.2) (layer "F.Cu") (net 1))
 (segment (start 58.7375 56.99125) (end 58.89625 57.15) (width 0.2) (layer "F.Cu") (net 1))
 (segment (start 58.7375 76.04125) (end 58.7375 56.99125) (width 0.2) (layer "F.Cu") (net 1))
 (segment (start 45.24375 47.625) (end 45.24375 38.1) (width 0.2) (layer "F.Cu") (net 1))
 (segment (start 58.89625 57.15) (end 59.53125 57.15) (width 0.2) (layer "F.Cu") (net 1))
 (segment (start 77.7875 39.525) (end 79.2125 38.1) (width 0.2) (layer "F.Cu") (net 1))
 (segment (start 50.00625 48.26) (end 45.87875 48.26) (width 0.2) (layer "F.Cu") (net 1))
 (segment (start 78.58125 42.8625) (end 79.2125 42.23125) (width 0.2) (layer "F.Cu") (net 3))
 (segment (start 85.725 38.1) (end 85.725 40.48125) (width 0.2) (layer "F.Cu") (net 3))
 (segment (start 85.725 40.48125) (end 83.34375 42.8625) (width 0.2) (layer "F.Cu") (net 3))
 (segment (start 51.125 34.6) (end 54.460375 31.264625) (width 0.2) (layer "F.Cu") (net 3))
 (segment (start 83.34375 42.8625) (end 78.58125 42.8625) (width 0.2) (layer "F.Cu") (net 3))
 (segment (start 54.460375 31.264625) (end 78.889625 31.264625) (width 0.2) (layer "F.Cu") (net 3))
 (segment (start 78.889625 31.264625) (end 85.725 38.1) (width 0.2) (layer "F.Cu") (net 3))
 (segment (start 51.125 38.1) (end 51.125 34.6) (width 0.2) (layer "F.Cu") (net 3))
 (segment (start 79.2125 42.23125) (end 79.2125 39.85) (width 0.2) (layer "F.Cu") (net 3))
 (segment (start 83.8135 38.749) (end 82.7125 39.85) (width 0.2) (layer "F.Cu") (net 4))
 (segment (start 79.777 33.3375) (end 83.8135 37.374) (width 0.2) (layer "F.Cu") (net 4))
 (segment (start 51.125 39.85) (end 65.8775 39.85) (width 0.2) (layer "F.Cu") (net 4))
 (segment (start 83.8135 37.374) (end 83.8135 38.749) (width 0.2) (layer "F.Cu") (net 4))
 (segment (start 65.8775 39.85) (end 72.39 33.3375) (width 0.2) (layer "F.Cu") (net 4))
 (segment (start 73.225 33.3375) (end 79.777 33.3375) (width 0.2) (layer "F.Cu") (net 4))
 (segment (start 73.453 43.05719) (end 73.453 47.5145) (width 0.2) (layer "B.Cu") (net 2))
 (segment (start 73.453 47.5145) (end 72.39 48.5775) (width 0.2) (layer "B.Cu") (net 2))
 (segment (start 69.48425 42.4345) (end 72.83031 42.4345) (width 0.2) (layer "B.Cu") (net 2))
 (segment (start 72.83031 42.4345) (end 73.453 43.05719) (width 0.2) (layer "B.Cu") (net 2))
 (segment (start 52.3875 59.53125) (end 69.48425 42.4345) (width 0.2) (layer "B.Cu") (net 2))
 (segment (start 71.4375 59.53125) (end 70.337501 58.431251) (width 0.2) (layer "B.Cu") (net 7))
 (segment (start 70.337501 58.431251) (end 70.337501 48.089999) (width 0.2) (layer "B.Cu") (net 7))
 (segment (start 70.337501 48.089999) (end 72.39 46.0375) (width 0.2) (layer "B.Cu") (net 7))
 (segment (start 72.39 43.4975) (end 73.225 43.4975) (width 0.2) (layer "F.Cu") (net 8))
 (segment (start 52.3875 78.58125) (end 52.3875 77.025616) (width 0.2) (layer "B.Cu") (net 8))
 (segment (start 52.3875 77.025616) (end 69.05625 60.356866) (width 0.2) (layer "B.Cu") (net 8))
 (segment (start 69.05625 60.356866) (end 69.05625 46.83125) (width 0.2) (layer "B.Cu") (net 8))
 (segment (start 69.05625 46.83125) (end 72.39 43.4975) (width 0.2) (layer "B.Cu") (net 8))
 (segment (start 73.854 42.4215) (end 72.39 40.9575) (width 0.2) (layer "B.Cu") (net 6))
 (segment (start 72.8385 58.950936) (end 73.854 57.935436) (width 0.2) (layer "B.Cu") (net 6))
 (segment (start 73.854 57.935436) (end 73.854 42.4215) (width 0.2) (layer "B.Cu") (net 6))
 (segment (start 71.4375 78.58125) (end 72.8385 77.18025) (width 0.2) (layer "B.Cu") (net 6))
 (segment (start 72.8385 77.18025) (end 72.8385 58.950936) (width 0.2) (layer "B.Cu") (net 6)))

